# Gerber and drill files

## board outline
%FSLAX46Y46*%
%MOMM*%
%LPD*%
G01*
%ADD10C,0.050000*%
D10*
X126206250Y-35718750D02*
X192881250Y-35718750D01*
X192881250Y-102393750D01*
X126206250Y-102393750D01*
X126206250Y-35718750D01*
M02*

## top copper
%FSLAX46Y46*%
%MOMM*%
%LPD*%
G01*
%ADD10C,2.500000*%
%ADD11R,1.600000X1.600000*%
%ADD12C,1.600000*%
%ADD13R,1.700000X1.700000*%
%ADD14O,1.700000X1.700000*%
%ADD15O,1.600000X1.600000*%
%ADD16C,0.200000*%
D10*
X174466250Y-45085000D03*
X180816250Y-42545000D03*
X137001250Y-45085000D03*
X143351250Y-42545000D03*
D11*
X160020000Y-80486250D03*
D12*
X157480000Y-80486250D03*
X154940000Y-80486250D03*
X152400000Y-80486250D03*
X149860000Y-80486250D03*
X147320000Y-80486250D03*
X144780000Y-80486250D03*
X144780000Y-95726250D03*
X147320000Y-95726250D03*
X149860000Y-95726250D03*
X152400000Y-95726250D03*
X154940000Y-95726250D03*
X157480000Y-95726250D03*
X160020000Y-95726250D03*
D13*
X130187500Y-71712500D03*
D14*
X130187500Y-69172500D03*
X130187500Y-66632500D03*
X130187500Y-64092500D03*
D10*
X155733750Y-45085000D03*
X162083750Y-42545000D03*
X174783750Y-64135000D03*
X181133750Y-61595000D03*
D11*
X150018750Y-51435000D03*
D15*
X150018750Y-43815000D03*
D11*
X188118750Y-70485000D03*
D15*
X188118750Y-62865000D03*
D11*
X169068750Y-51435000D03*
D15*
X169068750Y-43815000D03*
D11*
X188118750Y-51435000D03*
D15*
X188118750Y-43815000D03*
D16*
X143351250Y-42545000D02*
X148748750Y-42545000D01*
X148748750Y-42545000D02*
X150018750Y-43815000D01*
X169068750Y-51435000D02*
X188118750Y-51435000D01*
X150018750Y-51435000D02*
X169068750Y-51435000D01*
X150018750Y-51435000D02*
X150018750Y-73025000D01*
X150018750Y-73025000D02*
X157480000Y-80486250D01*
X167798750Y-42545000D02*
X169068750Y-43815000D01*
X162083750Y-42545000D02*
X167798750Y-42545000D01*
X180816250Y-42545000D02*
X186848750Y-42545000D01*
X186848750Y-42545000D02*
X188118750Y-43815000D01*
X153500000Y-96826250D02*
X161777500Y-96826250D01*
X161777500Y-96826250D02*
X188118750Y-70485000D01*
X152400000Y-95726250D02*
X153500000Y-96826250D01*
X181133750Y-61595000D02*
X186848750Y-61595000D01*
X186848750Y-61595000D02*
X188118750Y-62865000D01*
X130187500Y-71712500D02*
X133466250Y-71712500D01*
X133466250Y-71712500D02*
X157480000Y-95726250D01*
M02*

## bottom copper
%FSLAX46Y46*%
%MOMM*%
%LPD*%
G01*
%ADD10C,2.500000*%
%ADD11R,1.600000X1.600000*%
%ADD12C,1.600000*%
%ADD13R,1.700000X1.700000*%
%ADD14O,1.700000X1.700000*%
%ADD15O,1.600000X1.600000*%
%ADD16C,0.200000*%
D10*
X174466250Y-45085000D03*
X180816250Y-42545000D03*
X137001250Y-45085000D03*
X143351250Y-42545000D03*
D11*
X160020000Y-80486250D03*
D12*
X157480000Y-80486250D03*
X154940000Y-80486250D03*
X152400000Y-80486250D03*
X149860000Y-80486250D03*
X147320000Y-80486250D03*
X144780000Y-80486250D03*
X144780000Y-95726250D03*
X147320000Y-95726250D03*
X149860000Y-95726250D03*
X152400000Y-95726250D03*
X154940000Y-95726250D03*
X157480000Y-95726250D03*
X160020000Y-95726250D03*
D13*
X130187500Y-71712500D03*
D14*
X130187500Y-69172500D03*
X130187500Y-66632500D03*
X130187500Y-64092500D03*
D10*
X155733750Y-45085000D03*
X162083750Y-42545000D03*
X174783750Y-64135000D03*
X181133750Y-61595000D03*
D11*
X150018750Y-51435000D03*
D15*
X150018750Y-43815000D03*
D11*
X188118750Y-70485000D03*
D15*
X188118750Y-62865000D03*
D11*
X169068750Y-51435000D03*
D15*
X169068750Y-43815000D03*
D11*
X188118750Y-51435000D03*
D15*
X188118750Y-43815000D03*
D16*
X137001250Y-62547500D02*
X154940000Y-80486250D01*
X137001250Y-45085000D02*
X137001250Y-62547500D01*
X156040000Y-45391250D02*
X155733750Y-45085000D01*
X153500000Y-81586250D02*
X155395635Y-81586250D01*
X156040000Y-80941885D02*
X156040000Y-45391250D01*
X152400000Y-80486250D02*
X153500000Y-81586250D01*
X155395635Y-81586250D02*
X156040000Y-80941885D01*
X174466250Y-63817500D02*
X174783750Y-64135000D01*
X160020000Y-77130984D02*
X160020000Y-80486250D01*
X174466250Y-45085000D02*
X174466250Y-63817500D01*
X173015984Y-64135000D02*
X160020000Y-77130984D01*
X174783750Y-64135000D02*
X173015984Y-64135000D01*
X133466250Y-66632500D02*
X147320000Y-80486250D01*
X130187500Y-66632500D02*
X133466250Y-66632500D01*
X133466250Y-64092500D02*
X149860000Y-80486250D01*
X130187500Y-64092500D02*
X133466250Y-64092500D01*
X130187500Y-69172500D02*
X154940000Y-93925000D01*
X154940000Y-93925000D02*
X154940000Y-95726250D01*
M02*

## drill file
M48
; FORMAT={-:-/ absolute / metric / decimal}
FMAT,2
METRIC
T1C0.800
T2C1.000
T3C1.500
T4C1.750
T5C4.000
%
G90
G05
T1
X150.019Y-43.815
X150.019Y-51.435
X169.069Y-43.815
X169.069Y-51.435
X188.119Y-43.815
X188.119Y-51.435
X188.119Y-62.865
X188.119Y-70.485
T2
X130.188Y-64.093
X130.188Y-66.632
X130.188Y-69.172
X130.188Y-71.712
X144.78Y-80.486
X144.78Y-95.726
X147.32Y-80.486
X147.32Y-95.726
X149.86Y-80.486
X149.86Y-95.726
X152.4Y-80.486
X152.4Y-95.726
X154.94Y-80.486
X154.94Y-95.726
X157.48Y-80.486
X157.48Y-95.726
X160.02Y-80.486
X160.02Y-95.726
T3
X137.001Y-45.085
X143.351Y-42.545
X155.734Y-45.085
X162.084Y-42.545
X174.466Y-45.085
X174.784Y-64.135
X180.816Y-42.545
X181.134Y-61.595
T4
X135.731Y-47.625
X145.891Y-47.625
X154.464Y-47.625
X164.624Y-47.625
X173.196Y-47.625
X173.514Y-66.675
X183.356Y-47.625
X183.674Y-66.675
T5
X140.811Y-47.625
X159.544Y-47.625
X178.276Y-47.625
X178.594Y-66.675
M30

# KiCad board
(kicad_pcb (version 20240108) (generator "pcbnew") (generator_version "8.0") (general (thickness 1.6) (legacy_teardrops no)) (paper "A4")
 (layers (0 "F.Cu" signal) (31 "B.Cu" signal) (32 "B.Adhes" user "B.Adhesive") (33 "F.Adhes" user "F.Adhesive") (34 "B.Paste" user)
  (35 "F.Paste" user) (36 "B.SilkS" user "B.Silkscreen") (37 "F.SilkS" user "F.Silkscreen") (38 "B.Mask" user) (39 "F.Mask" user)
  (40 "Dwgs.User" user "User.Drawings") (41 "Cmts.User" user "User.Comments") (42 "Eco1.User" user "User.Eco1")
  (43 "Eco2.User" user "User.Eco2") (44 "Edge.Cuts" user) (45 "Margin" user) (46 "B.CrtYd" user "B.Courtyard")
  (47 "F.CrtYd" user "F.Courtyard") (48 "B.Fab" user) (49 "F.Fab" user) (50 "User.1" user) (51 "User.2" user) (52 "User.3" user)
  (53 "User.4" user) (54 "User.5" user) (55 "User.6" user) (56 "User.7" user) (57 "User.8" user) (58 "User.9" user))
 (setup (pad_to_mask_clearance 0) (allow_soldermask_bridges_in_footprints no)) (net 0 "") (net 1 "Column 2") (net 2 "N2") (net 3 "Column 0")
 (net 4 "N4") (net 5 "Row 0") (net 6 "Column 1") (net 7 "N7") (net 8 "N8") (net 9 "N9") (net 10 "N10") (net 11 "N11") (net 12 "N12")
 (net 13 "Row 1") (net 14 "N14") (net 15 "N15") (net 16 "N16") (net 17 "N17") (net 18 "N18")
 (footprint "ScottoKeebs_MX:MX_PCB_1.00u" (layer "F.Cu") (at 178.27625 47.625)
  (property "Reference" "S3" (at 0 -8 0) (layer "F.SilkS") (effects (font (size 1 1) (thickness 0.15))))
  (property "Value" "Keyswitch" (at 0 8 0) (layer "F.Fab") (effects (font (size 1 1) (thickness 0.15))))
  (pad "" np_thru_hole circle (at -5.08 0) (size 1.75 1.75) (drill 1.75) (layers "*.Cu" "*.Mask"))
  (pad "" np_thru_hole circle (at 0 0) (size 4 4) (drill 4) (layers "*.Cu" "*.Mask"))
  (pad "" np_thru_hole circle (at 5.08 0) (size 1.75 1.75) (drill 1.75) (layers "*.Cu" "*.Mask"))
  (pad "1" thru_hole circle (at -3.81 -2.54) (size 2.5 2.5) (drill 1.5) (layers "*.Cu" "*.Mask") (remove_unused_layers no)
   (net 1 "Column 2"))
  (pad "2" thru_hole circle (at 2.54 -5.08) (size 2.5 2.5) (drill 1.5) (layers "*.Cu" "*.Mask") (remove_unused_layers no) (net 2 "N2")))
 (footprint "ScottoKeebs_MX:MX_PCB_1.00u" (layer "F.Cu") (at 140.81125 47.625)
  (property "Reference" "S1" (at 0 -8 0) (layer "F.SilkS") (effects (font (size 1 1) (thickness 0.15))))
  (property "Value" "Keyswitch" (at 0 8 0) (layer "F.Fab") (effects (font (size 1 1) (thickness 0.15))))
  (pad "" np_thru_hole circle (at -5.08 0) (size 1.75 1.75) (drill 1.75) (layers "*.Cu" "*.Mask"))
  (pad "" np_thru_hole circle (at 0 0) (size 4 4) (drill 4) (layers "*.Cu" "*.Mask"))
  (pad "" np_thru_hole circle (at 5.08 0) (size 1.75 1.75) (drill 1.75) (layers "*.Cu" "*.Mask"))
  (pad "1" thru_hole circle (at -3.81 -2.54) (size 2.5 2.5) (drill 1.5) (layers "*.Cu" "*.Mask") (remove_unused_layers no)
   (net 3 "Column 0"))
  (pad "2" thru_hole circle (at 2.54 -5.08) (size 2.5 2.5) (drill 1.5) (layers "*.Cu" "*.Mask") (remove_unused_layers no) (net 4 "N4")))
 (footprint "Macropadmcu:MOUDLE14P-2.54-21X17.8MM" (layer "F.Cu") (at 152.4 88.10625)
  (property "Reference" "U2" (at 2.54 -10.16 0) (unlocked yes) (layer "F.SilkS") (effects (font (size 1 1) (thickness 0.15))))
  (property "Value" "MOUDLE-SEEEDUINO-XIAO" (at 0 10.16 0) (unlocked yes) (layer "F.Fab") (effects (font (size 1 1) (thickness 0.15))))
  (pad "1" thru_hole rect (at 7.62 -7.62) (size 1.6 1.6) (drill 1) (layers "*.Cu" "*.Mask") (remove_unused_layers no) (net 1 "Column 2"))
  (pad "2" thru_hole circle (at 5.08 -7.62) (size 1.6 1.6) (drill 1) (layers "*.Cu" "*.Mask") (remove_unused_layers no) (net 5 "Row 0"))
  (pad "3" thru_hole circle (at 2.54 -7.62) (size 1.6 1.6) (drill 1) (layers "*.Cu" "*.Mask") (remove_unused_layers no) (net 3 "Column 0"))
  (pad "4" thru_hole circle (at 0 -7.62) (size 1.6 1.6) (drill 1) (layers "*.Cu" "*.Mask") (remove_unused_layers no) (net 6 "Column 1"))
  (pad "5" thru_hole circle (at -2.54 -7.62) (size 1.6 1.6) (drill 1) (layers "*.Cu" "*.Mask") (remove_unused_layers no) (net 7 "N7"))
  (pad "6" thru_hole circle (at -5.08 -7.62) (size 1.6 1.6) (drill 1) (layers "*.Cu" "*.Mask") (remove_unused_layers no) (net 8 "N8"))
  (pad "7" thru_hole circle (at -7.62 -7.62) (size 1.6 1.6) (drill 1) (layers "*.Cu" "*.Mask") (remove_unused_layers no) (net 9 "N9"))
  (pad "8" thru_hole circle (at -7.62 7.62) (size 1.6 1.6) (drill 1) (layers "*.Cu" "*.Mask") (remove_unused_layers no) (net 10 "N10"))
  (pad "9" thru_hole circle (at -5.08 7.62) (size 1.6 1.6) (drill 1) (layers "*.Cu" "*.Mask") (remove_unused_layers no) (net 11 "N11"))
  (pad "10" thru_hole circle (at -2.54 7.62) (size 1.6 1.6) (drill 1) (layers "*.Cu" "*.Mask") (remove_unused_layers no) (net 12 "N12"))
  (pad "11" thru_hole circle (at 0 7.62) (size 1.6 1.6) (drill 1) (layers "*.Cu" "*.Mask") (remove_unused_layers no) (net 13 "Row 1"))
  (pad "12" thru_hole circle (at 2.54 7.62) (size 1.6 1.6) (drill 1) (layers "*.Cu" "*.Mask") (remove_unused_layers no) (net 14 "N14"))
  (pad "13" thru_hole circle (at 5.08 7.62) (size 1.6 1.6) (drill 1) (layers "*.Cu" "*.Mask") (remove_unused_layers no) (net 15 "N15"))
  (pad "14" thru_hole circle (at 7.62 7.62) (size 1.6 1.6) (drill 1) (layers "*.Cu" "*.Mask") (remove_unused_layers no) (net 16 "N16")))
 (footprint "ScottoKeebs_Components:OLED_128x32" (layer "F.Cu") (at 128.5875 61.9125)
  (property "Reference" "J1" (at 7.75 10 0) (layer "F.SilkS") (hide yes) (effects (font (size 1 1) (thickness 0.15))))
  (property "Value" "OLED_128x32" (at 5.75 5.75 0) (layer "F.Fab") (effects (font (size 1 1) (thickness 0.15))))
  (pad "1" thru_hole rect (at 1.6 9.8 180) (size 1.7 1.7) (drill 1) (layers "*.Cu" "*.Mask") (remove_unused_layers no) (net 15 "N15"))
  (pad "2" thru_hole oval (at 1.6 7.26 180) (size 1.7 1.7) (drill 1) (layers "*.Cu" "*.Mask") (remove_unused_layers no) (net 14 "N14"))
  (pad "3" thru_hole oval (at 1.6 4.72 180) (size 1.7 1.7) (drill 1) (layers "*.Cu" "*.Mask") (remove_unused_layers no) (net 8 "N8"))
  (pad "4" thru_hole oval (at 1.6 2.18 180) (size 1.7 1.7) (drill 1) (layers "*.Cu" "*.Mask") (remove_unused_layers no) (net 7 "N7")))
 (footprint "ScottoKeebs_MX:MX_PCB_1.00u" (layer "F.Cu") (at 159.54375 47.625)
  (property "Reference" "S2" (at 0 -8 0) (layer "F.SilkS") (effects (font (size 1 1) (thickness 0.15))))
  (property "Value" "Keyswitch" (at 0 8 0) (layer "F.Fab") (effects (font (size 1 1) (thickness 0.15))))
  (pad "" np_thru_hole circle (at -5.08 0) (size 1.75 1.75) (drill 1.75) (layers "*.Cu" "*.Mask"))
  (pad "" np_thru_hole circle (at 0 0) (size 4 4) (drill 4) (layers "*.Cu" "*.Mask"))
  (pad "" np_thru_hole circle (at 5.08 0) (size 1.75 1.75) (drill 1.75) (layers "*.Cu" "*.Mask"))
  (pad "1" thru_hole circle (at -3.81 -2.54) (size 2.5 2.5) (drill 1.5) (layers "*.Cu" "*.Mask") (remove_unused_layers no)
   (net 6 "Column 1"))
  (pad "2" thru_hole circle (at 2.54 -5.08) (size 2.5 2.5) (drill 1.5) (layers "*.Cu" "*.Mask") (remove_unused_layers no) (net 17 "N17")))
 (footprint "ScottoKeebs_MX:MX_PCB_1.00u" (layer "F.Cu") (at 178.59375 66.675)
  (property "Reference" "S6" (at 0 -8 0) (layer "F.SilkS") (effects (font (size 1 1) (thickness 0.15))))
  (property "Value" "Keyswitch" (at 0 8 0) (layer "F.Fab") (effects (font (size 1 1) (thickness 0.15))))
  (pad "" np_thru_hole circle (at -5.08 0) (size 1.75 1.75) (drill 1.75) (layers "*.Cu" "*.Mask"))
  (pad "" np_thru_hole circle (at 0 0) (size 4 4) (drill 4) (layers "*.Cu" "*.Mask"))
  (pad "" np_thru_hole circle (at 5.08 0) (size 1.75 1.75) (drill 1.75) (layers "*.Cu" "*.Mask"))
  (pad "1" thru_hole circle (at -3.81 -2.54) (size 2.5 2.5) (drill 1.5) (layers "*.Cu" "*.Mask") (remove_unused_layers no)
   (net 1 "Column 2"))
  (pad "2" thru_hole circle (at 2.54 -5.08) (size 2.5 2.5) (drill 1.5) (layers "*.Cu" "*.Mask") (remove_unused_layers no) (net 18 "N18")))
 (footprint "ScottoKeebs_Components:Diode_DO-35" (layer "B.Cu") (at 150.01875 51.435 90)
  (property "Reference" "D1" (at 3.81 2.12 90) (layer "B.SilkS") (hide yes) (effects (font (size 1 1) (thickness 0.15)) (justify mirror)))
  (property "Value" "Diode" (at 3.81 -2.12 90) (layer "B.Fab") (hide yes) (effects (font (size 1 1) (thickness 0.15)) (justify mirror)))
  (pad "1" thru_hole rect (at 0 0 90) (size 1.6 1.6) (drill 0.8) (layers "*.Cu" "*.Mask") (remove_unused_layers no) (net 5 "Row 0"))
  (pad "2" thru_hole oval (at 7.62 0 90) (size 1.6 1.6) (drill 0.8) (layers "*.Cu" "*.Mask") (remove_unused_layers no) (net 4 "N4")))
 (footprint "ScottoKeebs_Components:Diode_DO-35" (layer "B.Cu") (at 188.11875 70.485 90)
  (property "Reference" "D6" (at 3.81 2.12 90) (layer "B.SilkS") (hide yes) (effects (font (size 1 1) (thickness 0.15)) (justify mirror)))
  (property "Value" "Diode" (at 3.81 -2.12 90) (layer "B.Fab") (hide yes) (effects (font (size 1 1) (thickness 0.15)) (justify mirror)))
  (pad "1" thru_hole rect (at 0 0 90) (size 1.6 1.6) (drill 0.8) (layers "*.Cu" "*.Mask") (remove_unused_layers no) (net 13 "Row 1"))
  (pad "2" thru_hole oval (at 7.62 0 90) (size 1.6 1.6) (drill 0.8) (layers "*.Cu" "*.Mask") (remove_unused_layers no) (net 18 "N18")))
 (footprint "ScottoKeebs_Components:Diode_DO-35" (layer "B.Cu") (at 169.06875 51.435 90)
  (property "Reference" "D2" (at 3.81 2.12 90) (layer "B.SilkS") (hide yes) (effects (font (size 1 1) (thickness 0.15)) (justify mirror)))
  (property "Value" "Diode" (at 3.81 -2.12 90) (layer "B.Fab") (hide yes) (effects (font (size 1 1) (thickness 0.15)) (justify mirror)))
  (pad "1" thru_hole rect (at 0 0 90) (size 1.6 1.6) (drill 0.8) (layers "*.Cu" "*.Mask") (remove_unused_layers no) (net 5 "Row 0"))
  (pad "2" thru_hole oval (at 7.62 0 90) (size 1.6 1.6) (drill 0.8) (layers "*.Cu" "*.Mask") (remove_unused_layers no) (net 17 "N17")))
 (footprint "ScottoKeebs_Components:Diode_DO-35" (layer "B.Cu") (at 188.11875 51.435 90)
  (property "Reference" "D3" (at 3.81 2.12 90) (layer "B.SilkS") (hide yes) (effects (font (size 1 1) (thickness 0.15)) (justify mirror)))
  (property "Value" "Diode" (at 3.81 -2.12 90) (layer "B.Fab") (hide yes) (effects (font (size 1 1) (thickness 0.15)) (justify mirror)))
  (pad "1" thru_hole rect (at 0 0 90) (size 1.6 1.6) (drill 0.8) (layers "*.Cu" "*.Mask") (remove_unused_layers no) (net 5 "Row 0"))
  (pad "2" thru_hole oval (at 7.62 0 90) (size 1.6 1.6) (drill 0.8) (layers "*.Cu" "*.Mask") (remove_unused_layers no) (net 2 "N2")))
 (gr_rect (start 126.20625 35.71875) (end 192.88125 102.39375) (stroke (width 0.05) (type default)) (fill none) (layer "Edge.Cuts"))
 (segment (start 143.35125 42.545) (end 148.74875 42.545) (width 0.2) (layer "F.Cu") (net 4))
 (segment (start 148.74875 42.545) (end 150.01875 43.815) (width 0.2) (layer "F.Cu") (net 4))
 (segment (start 169.06875 51.435) (end 188.11875 51.435) (width 0.2) (layer "F.Cu") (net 5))
 (segment (start 150.01875 51.435) (end 169.06875 51.435) (width 0.2) (layer "F.Cu") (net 5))
 (segment (start 150.01875 51.435) (end 150.01875 73.025) (width 0.2) (layer "F.Cu") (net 5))
 (segment (start 150.01875 73.025) (end 157.48 80.48625) (width 0.2) (layer "F.Cu") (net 5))
 (segment (start 167.79875 42.545) (end 169.06875 43.815) (width 0.2) (layer "F.Cu") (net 17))
 (segment (start 162.08375 42.545) (end 167.79875 42.545) (width 0.2) (layer "F.Cu") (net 17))
 (segment (start 180.81625 42.545) (end 186.84875 42.545) (width 0.2) (layer "F.Cu") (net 2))
 (segment (start 186.84875 42.545) (end 188.11875 43.815) (width 0.2) (layer "F.Cu") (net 2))
 (segment (start 153.5 96.82625) (end 161.7775 96.82625) (width 0.2) (layer "F.Cu") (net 13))
 (segment (start 161.7775 96.82625) (end 188.11875 70.485) (width 0.2) (layer "F.Cu") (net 13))
 (segment (start 152.4 95.72625) (end 153.5 96.82625) (width 0.2) (layer "F.Cu") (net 13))
 (segment (start 181.13375 61.595) (end 186.84875 61.595) (width 0.2) (layer "F.Cu") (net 18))
 (segment (start 186.84875 61.595) (end 188.11875 62.865) (width 0.2) (layer "F.Cu") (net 18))
 (segment (start 137.00125 62.5475) (end 154.94 80.48625) (width 0.2) (layer "B.Cu") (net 3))
 (segment (start 137.00125 45.085) (end 137.00125 62.5475) (width 0.2) (layer "B.Cu") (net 3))
 (segment (start 156.04 45.39125) (end 155.73375 45.085) (width 0.2) (layer "B.Cu") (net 6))
 (segment (start 153.5 81.58625) (end 155.395635 81.58625) (width 0.2) (layer "B.Cu") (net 6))
 (segment (start 156.04 80.941885) (end 156.04 45.39125) (width 0.2) (layer "B.Cu") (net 6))
 (segment (start 152.4 80.48625) (end 153.5 81.58625) (width 0.2) (layer "B.Cu") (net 6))
 (segment (start 155.395635 81.58625) (end 156.04 80.941885) (width 0.2) (layer "B.Cu") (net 6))
 (segment (start 174.46625 63.8175) (end 174.78375 64.135) (width 0.2) (layer "B.Cu") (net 1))
 (segment (start 160.02 77.130984) (end 160.02 80.48625) (width 0.2) (layer "B.Cu") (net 1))
 (segment (start 174.46625 45.085) (end 174.46625 63.8175) (width 0.2) (layer "B.Cu") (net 1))
 (segment (start 173.015984 64.135) (end 160.02 77.130984) (width 0.2) (layer "B.Cu") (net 1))
 (segment (start 174.78375 64.135) (end 173.015984 64.135) (width 0.2) (layer "B.Cu") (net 1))
 (segment (start 130.1875 71.7125) (end 133.46625 71.7125) (width 0.2) (layer "F.Cu") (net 15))
 (segment (start 133.46625 71.7125) (end 157.48 95.72625) (width 0.2) (layer "F.Cu") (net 15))
 (segment (start 133.46625 66.6325) (end 147.32 80.48625) (width 0.2) (layer "B.Cu") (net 8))
 (segment (start 130.1875 66.6325) (end 133.46625 66.6325) (width 0.2) (layer "B.Cu") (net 8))
 (segment (start 133.46625 64.0925) (end 149.86 80.48625) (width 0.2) (layer "B.Cu") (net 7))
 (segment (start 130.1875 64.0925) (end 133.46625 64.0925) (width 0.2) (layer "B.Cu") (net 7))
 (segment (start 130.1875 69.1725) (end 154.94 93.925) (width 0.2) (layer "B.Cu") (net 14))
 (segment (start 154.94 93.925) (end 154.94 95.72625) (width 0.2) (layer "B.Cu") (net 14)))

